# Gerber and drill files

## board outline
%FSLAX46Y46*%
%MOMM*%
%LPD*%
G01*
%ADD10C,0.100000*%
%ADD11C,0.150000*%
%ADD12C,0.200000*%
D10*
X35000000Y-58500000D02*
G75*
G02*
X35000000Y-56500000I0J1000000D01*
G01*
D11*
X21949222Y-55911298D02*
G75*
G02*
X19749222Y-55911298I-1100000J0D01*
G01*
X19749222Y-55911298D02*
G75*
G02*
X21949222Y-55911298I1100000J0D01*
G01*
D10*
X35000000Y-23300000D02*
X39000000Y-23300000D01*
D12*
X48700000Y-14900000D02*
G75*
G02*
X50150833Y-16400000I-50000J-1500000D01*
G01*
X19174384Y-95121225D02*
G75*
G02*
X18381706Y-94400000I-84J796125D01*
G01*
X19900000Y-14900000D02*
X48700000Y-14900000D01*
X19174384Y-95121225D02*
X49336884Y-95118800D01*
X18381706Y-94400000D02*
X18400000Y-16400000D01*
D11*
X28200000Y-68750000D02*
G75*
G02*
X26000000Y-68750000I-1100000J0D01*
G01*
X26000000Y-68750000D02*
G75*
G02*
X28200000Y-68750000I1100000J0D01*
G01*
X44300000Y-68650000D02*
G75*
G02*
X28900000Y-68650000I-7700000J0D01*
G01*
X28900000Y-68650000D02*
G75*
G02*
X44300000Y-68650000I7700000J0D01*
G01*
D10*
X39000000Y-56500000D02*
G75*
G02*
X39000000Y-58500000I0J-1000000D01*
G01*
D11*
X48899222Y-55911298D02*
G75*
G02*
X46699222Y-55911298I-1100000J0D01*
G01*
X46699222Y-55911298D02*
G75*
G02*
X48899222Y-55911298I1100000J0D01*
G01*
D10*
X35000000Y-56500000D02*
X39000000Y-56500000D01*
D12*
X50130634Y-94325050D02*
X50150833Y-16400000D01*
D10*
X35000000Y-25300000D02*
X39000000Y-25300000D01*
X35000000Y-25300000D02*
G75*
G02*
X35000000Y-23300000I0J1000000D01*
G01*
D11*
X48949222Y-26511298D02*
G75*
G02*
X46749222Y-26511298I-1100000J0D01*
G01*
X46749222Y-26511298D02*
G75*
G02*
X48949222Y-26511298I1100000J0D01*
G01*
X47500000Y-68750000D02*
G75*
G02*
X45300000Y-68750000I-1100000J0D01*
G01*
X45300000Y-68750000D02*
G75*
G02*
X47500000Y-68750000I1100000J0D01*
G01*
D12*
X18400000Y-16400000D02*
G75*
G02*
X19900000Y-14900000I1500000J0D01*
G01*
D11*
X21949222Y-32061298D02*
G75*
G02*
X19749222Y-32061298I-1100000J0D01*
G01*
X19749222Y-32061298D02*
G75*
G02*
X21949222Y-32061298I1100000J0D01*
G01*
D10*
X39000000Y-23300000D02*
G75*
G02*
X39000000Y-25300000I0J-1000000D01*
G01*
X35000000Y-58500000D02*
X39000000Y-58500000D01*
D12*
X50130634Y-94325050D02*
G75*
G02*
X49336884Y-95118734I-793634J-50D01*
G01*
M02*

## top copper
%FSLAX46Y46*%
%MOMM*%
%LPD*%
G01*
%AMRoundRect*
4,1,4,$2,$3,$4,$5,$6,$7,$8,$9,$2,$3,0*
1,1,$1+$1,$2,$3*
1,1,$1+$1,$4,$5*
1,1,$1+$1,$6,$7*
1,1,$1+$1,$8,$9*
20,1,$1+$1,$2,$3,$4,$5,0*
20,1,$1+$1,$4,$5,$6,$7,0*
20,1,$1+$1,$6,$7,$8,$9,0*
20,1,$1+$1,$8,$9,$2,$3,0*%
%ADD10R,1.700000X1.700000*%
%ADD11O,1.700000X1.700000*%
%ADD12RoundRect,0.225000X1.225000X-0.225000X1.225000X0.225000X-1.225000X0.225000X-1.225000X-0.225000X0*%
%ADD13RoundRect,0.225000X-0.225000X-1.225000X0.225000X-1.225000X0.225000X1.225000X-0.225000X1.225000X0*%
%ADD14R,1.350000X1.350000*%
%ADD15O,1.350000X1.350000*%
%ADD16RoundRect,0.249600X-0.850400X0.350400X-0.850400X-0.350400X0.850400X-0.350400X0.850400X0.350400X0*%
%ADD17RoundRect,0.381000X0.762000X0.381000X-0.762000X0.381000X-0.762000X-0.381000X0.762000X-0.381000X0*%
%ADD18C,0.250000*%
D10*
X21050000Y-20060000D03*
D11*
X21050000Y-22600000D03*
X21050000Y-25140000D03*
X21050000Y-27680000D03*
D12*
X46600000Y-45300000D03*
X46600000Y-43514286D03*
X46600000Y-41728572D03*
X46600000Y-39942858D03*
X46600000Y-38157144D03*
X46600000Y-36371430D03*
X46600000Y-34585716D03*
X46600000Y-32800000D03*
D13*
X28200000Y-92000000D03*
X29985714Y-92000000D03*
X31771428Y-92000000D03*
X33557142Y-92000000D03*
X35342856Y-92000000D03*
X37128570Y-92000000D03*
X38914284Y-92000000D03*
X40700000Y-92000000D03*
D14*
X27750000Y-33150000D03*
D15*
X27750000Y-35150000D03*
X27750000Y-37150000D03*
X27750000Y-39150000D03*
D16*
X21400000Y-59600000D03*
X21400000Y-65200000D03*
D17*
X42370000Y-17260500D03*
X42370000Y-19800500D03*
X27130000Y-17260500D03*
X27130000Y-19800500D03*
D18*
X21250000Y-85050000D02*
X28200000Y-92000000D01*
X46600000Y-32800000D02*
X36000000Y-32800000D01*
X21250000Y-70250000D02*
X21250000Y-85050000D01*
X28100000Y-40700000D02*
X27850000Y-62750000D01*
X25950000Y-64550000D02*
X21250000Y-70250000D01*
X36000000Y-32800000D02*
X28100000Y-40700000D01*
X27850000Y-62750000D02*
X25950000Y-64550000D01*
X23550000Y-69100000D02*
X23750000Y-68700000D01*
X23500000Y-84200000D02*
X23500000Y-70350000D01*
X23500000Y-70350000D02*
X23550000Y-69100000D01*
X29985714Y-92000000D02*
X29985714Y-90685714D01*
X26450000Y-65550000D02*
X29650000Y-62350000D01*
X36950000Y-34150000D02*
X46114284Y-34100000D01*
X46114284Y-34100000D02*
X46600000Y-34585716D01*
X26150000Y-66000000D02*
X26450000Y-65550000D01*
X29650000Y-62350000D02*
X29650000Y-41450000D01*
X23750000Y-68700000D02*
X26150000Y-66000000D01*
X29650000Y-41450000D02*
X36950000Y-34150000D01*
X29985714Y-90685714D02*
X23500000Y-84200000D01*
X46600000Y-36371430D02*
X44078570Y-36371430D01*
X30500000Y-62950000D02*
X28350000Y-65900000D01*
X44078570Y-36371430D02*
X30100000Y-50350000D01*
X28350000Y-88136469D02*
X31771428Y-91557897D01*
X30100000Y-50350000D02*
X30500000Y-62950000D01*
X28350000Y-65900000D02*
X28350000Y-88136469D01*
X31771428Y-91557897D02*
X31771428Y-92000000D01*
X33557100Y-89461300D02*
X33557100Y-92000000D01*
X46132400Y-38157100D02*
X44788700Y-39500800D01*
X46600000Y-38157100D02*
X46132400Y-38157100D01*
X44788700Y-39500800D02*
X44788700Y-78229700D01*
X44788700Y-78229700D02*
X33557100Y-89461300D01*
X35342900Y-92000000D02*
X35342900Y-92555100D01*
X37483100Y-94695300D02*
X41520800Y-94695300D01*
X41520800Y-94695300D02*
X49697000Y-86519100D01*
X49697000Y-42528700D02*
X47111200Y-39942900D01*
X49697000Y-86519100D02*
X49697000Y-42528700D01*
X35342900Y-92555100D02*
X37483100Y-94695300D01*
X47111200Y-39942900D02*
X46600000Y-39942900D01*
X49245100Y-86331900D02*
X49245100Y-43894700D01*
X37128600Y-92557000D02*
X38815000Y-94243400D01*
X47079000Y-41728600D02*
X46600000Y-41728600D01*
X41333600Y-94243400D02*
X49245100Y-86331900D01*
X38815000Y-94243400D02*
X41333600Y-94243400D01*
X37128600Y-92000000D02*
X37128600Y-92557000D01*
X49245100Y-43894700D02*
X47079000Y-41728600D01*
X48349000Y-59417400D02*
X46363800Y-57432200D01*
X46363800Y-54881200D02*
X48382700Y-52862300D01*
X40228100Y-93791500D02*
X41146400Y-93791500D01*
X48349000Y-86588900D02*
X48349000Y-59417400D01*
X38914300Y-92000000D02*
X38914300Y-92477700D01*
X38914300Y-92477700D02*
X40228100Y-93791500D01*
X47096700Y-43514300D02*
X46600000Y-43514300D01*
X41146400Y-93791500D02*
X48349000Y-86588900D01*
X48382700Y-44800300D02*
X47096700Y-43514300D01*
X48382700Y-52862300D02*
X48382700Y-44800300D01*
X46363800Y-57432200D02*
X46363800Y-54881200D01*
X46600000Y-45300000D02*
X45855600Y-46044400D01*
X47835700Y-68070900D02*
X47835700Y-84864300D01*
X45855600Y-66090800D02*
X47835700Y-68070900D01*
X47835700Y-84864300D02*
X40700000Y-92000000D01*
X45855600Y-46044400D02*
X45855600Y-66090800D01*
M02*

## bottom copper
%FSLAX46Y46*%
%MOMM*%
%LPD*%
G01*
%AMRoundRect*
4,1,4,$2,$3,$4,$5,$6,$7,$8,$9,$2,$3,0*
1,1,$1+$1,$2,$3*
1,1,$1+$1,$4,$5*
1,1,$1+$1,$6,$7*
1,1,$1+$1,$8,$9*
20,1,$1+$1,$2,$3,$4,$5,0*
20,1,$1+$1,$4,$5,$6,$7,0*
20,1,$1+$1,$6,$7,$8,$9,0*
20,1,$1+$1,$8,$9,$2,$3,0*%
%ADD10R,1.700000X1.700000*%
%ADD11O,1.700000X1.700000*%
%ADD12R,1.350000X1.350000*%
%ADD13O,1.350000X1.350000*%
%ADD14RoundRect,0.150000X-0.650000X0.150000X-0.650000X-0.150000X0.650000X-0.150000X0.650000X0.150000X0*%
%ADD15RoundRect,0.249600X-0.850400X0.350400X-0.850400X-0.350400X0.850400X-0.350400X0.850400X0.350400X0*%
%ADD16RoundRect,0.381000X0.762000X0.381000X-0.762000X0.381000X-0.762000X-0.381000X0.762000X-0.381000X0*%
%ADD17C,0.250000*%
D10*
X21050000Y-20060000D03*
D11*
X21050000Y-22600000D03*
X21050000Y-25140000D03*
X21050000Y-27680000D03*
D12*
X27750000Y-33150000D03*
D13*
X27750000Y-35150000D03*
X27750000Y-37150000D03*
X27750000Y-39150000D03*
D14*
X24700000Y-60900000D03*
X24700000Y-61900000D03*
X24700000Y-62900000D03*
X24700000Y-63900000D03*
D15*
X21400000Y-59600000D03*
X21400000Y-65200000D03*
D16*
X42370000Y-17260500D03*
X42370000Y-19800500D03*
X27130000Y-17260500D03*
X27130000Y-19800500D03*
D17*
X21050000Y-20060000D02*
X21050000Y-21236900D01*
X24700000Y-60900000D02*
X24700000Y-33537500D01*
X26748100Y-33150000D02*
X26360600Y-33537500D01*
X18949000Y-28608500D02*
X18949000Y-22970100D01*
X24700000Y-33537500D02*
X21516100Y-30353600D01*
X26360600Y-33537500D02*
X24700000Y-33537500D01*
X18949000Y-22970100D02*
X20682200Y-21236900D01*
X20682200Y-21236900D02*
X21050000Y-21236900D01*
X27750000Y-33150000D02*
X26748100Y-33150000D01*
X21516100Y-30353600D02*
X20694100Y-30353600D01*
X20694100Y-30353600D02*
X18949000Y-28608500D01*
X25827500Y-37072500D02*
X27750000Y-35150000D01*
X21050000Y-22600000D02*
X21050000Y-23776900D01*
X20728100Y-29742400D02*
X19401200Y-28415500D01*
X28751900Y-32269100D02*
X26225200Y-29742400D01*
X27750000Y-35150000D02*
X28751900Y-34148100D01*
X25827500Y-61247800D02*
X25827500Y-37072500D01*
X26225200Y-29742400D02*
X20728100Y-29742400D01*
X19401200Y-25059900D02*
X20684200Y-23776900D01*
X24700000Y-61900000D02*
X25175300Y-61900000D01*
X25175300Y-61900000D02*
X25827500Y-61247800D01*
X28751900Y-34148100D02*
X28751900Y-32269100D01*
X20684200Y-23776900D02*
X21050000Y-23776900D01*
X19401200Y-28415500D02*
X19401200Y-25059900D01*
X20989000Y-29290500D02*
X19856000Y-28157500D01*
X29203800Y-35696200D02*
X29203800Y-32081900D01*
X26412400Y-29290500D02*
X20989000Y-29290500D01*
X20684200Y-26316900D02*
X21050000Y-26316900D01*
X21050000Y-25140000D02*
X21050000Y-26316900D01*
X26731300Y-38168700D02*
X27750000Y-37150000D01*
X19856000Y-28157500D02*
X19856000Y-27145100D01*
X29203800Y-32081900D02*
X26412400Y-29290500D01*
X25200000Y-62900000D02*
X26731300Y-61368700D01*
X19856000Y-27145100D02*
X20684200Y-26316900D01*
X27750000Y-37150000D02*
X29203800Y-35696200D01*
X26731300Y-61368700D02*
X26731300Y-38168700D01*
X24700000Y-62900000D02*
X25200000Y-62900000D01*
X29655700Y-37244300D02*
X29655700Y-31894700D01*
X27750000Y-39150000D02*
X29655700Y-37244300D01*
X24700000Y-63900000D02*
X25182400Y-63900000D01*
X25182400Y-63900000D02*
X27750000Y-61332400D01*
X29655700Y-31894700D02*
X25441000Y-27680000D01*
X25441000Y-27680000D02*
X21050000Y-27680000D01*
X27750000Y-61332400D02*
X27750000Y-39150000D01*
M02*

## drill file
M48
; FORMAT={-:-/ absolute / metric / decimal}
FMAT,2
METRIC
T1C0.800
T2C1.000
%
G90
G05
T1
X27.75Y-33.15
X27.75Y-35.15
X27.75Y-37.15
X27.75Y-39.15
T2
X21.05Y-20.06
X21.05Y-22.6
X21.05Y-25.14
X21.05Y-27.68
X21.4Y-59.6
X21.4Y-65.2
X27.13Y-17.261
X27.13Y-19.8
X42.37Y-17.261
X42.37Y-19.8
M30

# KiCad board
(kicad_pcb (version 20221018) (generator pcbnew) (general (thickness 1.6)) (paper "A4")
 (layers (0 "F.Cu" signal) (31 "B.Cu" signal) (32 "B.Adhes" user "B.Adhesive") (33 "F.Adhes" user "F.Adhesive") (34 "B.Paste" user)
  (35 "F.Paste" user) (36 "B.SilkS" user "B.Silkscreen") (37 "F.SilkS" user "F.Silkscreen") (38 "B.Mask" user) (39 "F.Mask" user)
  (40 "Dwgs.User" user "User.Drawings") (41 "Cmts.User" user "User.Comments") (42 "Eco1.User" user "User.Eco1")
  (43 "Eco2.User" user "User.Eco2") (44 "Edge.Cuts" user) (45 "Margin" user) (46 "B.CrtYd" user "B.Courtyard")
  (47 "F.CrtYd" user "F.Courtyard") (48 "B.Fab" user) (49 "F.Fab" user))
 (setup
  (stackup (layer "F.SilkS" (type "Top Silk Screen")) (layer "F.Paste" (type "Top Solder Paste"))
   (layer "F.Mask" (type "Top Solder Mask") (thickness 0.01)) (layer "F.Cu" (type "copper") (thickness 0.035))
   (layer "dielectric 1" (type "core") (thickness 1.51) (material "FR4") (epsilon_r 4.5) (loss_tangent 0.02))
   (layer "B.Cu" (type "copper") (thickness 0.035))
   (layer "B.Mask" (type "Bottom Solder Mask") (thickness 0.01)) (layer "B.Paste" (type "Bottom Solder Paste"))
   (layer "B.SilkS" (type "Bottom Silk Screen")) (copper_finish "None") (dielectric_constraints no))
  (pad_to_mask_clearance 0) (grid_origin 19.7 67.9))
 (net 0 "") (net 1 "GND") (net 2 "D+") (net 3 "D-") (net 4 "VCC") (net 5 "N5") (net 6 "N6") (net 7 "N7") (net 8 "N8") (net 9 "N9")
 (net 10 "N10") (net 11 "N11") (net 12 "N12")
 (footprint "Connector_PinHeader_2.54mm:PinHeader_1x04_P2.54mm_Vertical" (layer "F.Cu") (at 21.05 20.06)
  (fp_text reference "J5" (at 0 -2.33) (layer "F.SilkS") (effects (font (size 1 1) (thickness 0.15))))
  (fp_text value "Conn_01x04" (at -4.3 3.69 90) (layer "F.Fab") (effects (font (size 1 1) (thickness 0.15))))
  (pad "1" thru_hole rect (at 0 0) (size 1.7 1.7) (drill 1) (layers "*.Cu" "*.Mask") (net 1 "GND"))
  (pad "2" thru_hole oval (at 0 2.54) (size 1.7 1.7) (drill 1) (layers "*.Cu" "*.Mask") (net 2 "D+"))
  (pad "3" thru_hole oval (at 0 5.08) (size 1.7 1.7) (drill 1) (layers "*.Cu" "*.Mask") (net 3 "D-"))
  (pad "4" thru_hole oval (at 0 7.62) (size 1.7 1.7) (drill 1) (layers "*.Cu" "*.Mask") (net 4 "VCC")))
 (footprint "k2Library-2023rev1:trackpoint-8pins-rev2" (layer "F.Cu") (at 44.1 38.55 90)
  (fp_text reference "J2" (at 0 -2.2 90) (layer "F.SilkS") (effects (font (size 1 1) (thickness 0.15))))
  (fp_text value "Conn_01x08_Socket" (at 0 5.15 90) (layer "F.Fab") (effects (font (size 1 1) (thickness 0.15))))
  (pad "1" smd roundrect (at -6.75 2.5 90) (size 0.9 2.9) (layers "F.Cu" "F.Paste" "F.Mask") (roundrect_rratio 0.25) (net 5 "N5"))
  (pad "2" smd roundrect (at -4.964286 2.5 90) (size 0.9 2.9) (layers "F.Cu" "F.Paste" "F.Mask") (roundrect_rratio 0.25) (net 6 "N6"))
  (pad "3" smd roundrect (at -3.178572 2.5 90) (size 0.9 2.9) (layers "F.Cu" "F.Paste" "F.Mask") (roundrect_rratio 0.25) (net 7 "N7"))
  (pad "4" smd roundrect (at -1.392858 2.5 90) (size 0.9 2.9) (layers "F.Cu" "F.Paste" "F.Mask") (roundrect_rratio 0.25) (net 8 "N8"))
  (pad "5" smd roundrect (at 0.392856 2.5 90) (size 0.9 2.9) (layers "F.Cu" "F.Paste" "F.Mask") (roundrect_rratio 0.25) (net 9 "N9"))
  (pad "6" smd roundrect (at 2.17857 2.5 90) (size 0.9 2.9) (layers "F.Cu" "F.Paste" "F.Mask") (roundrect_rratio 0.25) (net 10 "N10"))
  (pad "7" smd roundrect (at 3.964284 2.5 90) (size 0.9 2.9) (layers "F.Cu" "F.Paste" "F.Mask") (roundrect_rratio 0.25) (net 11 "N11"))
  (pad "8" smd roundrect (at 5.75 2.5 90) (size 0.9 2.9) (layers "F.Cu" "F.Paste" "F.Mask") (roundrect_rratio 0.25) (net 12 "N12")))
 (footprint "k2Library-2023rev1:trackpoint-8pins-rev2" (layer "F.Cu") (at 34.95 89.5)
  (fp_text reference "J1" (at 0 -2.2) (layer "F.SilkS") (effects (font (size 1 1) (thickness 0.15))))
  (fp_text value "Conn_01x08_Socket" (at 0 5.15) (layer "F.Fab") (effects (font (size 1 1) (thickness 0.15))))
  (pad "1" smd roundrect (at -6.75 2.5) (size 0.9 2.9) (layers "F.Cu" "F.Paste" "F.Mask") (roundrect_rratio 0.25) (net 12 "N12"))
  (pad "2" smd roundrect (at -4.964286 2.5) (size 0.9 2.9) (layers "F.Cu" "F.Paste" "F.Mask") (roundrect_rratio 0.25) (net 11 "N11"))
  (pad "3" smd roundrect (at -3.178572 2.5) (size 0.9 2.9) (layers "F.Cu" "F.Paste" "F.Mask") (roundrect_rratio 0.25) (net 10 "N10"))
  (pad "4" smd roundrect (at -1.392858 2.5) (size 0.9 2.9) (layers "F.Cu" "F.Paste" "F.Mask") (roundrect_rratio 0.25) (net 9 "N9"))
  (pad "5" smd roundrect (at 0.392856 2.5) (size 0.9 2.9) (layers "F.Cu" "F.Paste" "F.Mask") (roundrect_rratio 0.25) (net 8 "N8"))
  (pad "6" smd roundrect (at 2.17857 2.5) (size 0.9 2.9) (layers "F.Cu" "F.Paste" "F.Mask") (roundrect_rratio 0.25) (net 7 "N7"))
  (pad "7" smd roundrect (at 3.964284 2.5) (size 0.9 2.9) (layers "F.Cu" "F.Paste" "F.Mask") (roundrect_rratio 0.25) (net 6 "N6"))
  (pad "8" smd roundrect (at 5.75 2.5) (size 0.9 2.9) (layers "F.Cu" "F.Paste" "F.Mask") (roundrect_rratio 0.25) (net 5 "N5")))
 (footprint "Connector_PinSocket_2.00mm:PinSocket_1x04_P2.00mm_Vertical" (layer "B.Cu") (at 27.75 33.15 180)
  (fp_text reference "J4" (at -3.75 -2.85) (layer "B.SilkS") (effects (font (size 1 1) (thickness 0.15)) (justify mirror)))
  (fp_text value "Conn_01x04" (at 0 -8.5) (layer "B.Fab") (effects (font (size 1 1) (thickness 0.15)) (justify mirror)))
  (pad "1" thru_hole rect (at 0 0 180) (size 1.35 1.35) (drill 0.8) (layers "*.Cu" "*.Mask") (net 1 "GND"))
  (pad "2" thru_hole oval (at 0 -2 180) (size 1.35 1.35) (drill 0.8) (layers "*.Cu" "*.Mask") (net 2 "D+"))
  (pad "3" thru_hole oval (at 0 -4 180) (size 1.35 1.35) (drill 0.8) (layers "*.Cu" "*.Mask") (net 3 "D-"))
  (pad "4" thru_hole oval (at 0 -6 180) (size 1.35 1.35) (drill 0.8) (layers "*.Cu" "*.Mask") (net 4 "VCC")))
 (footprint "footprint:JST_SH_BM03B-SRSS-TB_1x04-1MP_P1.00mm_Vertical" (layer "B.Cu") (at 22.9 62.4 -90)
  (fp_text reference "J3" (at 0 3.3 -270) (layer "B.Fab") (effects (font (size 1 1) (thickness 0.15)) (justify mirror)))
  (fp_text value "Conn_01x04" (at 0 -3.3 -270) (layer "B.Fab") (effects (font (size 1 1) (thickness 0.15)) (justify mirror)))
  (pad "1" smd roundrect (at -1.5 -1.8 270) (size 0.6 1.6) (layers "B.Cu" "B.Paste" "B.Mask") (roundrect_rratio 0.25) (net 1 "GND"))
  (pad "2" smd roundrect (at -0.5 -1.8 270) (size 0.6 1.6) (layers "B.Cu" "B.Paste" "B.Mask") (roundrect_rratio 0.25) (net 2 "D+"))
  (pad "3" smd roundrect (at 0.5 -1.8 270) (size 0.6 1.6) (layers "B.Cu" "B.Paste" "B.Mask") (roundrect_rratio 0.25) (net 3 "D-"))
  (pad "4" smd roundrect (at 1.5 -1.8 270) (size 0.6 1.6) (layers "B.Cu" "B.Paste" "B.Mask") (roundrect_rratio 0.25) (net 4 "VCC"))
  (pad "MP" thru_hole roundrect (at -2.8 1.5 270) (size 1.2 2.2) (drill 1) (layers "*.Cu" "*.Mask") (roundrect_rratio 0.208))
  (pad "MP" thru_hole roundrect (at 2.8 1.5 270) (size 1.2 2.2) (drill 1) (layers "*.Cu" "*.Mask") (roundrect_rratio 0.208)))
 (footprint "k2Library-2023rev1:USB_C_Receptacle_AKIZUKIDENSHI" (layer "B.Cu") (at 34.75 22.6005 180)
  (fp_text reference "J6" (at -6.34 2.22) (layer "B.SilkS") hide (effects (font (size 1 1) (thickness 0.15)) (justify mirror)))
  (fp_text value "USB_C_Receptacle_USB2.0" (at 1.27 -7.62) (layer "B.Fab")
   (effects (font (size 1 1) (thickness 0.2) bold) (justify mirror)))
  (pad "1" thru_hole roundrect (at -7.62 5.34 180) (size 2.286 1.524) (drill 1) (layers "*.Cu" "*.Mask") (roundrect_rratio 0.25)
   (thermal_bridge_angle 45))
  (pad "2" thru_hole roundrect (at -7.62 2.8 180) (size 2.286 1.524) (drill 1) (layers "*.Cu" "*.Mask") (roundrect_rratio 0.25)
   (thermal_bridge_angle 45))
  (pad "3" thru_hole roundrect (at 7.62 5.34 180) (size 2.286 1.524) (drill 1) (layers "*.Cu" "*.Mask") (roundrect_rratio 0.25)
   (thermal_bridge_angle 45))
  (pad "4" thru_hole roundrect (at 7.62 2.8 180) (size 2.286 1.524) (drill 1) (layers "*.Cu" "*.Mask") (roundrect_rratio 0.25)
   (thermal_bridge_angle 45)))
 (gr_arc (start 35 58.5) (mid 34 57.5) (end 35 56.5) (stroke (width 0.1) (type default)) (layer "Edge.Cuts"))
 (gr_circle (center 20.849222 55.911298) (end 21.949222 55.911298) (stroke (width 0.15) (type default)) (fill none) (layer "Edge.Cuts"))
 (gr_line (start 35 23.3) (end 39 23.3) (stroke (width 0.1) (type default)) (layer "Edge.Cuts"))
 (gr_arc (start 48.7 14.9) (mid 49.728781 15.356578) (end 50.150833 16.4) (stroke (width 0.2) (type solid)) (layer "Edge.Cuts"))
 (gr_arc (start 19.174384 95.121225) (mid 18.638521 94.91396) (end 18.381706 94.4) (stroke (width 0.2) (type solid)) (layer "Edge.Cuts"))
 (gr_line (start 19.9 14.9) (end 48.7 14.9) (stroke (width 0.2) (type solid)) (layer "Edge.Cuts"))
 (gr_line (start 19.174384 95.121225) (end 49.336884 95.1188) (stroke (width 0.2) (type solid)) (layer "Edge.Cuts"))
 (gr_line (start 18.381706 94.4) (end 18.4 16.4) (stroke (width 0.2) (type solid)) (layer "Edge.Cuts"))
 (gr_circle (center 27.1 68.75) (end 28.2 68.75) (stroke (width 0.15) (type solid)) (fill none) (layer "Edge.Cuts"))
 (gr_circle (center 36.6 68.65) (end 44.3 68.65) (stroke (width 0.15) (type solid)) (fill none) (layer "Edge.Cuts"))
 (gr_arc (start 39 56.5) (mid 40 57.5) (end 39 58.5) (stroke (width 0.1) (type default)) (layer "Edge.Cuts"))
 (gr_circle (center 47.799222 55.911298) (end 48.899222 55.911298) (stroke (width 0.15) (type default)) (fill none) (layer "Edge.Cuts"))
 (gr_line (start 35 56.5) (end 39 56.5) (stroke (width 0.1) (type default)) (layer "Edge.Cuts"))
 (gr_line (start 50.130634 94.32505) (end 50.150833 16.4) (stroke (width 0.2) (type solid)) (layer "Edge.Cuts"))
 (gr_line (start 35 25.3) (end 39 25.3) (stroke (width 0.1) (type default)) (layer "Edge.Cuts"))
 (gr_arc (start 35 25.3) (mid 34 24.3) (end 35 23.3) (stroke (width 0.1) (type default)) (layer "Edge.Cuts"))
 (gr_circle (center 47.849222 26.511298) (end 48.949222 26.511298) (stroke (width 0.15) (type default)) (fill none) (layer "Edge.Cuts"))
 (gr_circle (center 46.4 68.75) (end 47.5 68.75) (stroke (width 0.15) (type solid)) (fill none) (layer "Edge.Cuts"))
 (gr_arc (start 18.4 16.4) (mid 18.83934 15.33934) (end 19.9 14.9) (stroke (width 0.2) (type solid)) (layer "Edge.Cuts"))
 (gr_circle (center 20.849222 32.061298) (end 21.949222 32.061298) (stroke (width 0.15) (type default)) (fill none) (layer "Edge.Cuts"))
 (gr_arc (start 39 23.3) (mid 40 24.3) (end 39 25.3) (stroke (width 0.1) (type default)) (layer "Edge.Cuts"))
 (gr_line (start 35 58.5) (end 39 58.5) (stroke (width 0.1) (type default)) (layer "Edge.Cuts"))
 (gr_arc (start 50.130634 94.32505) (mid 49.898174 94.88634) (end 49.336884 95.1188) (stroke (width 0.2) (type solid)) (layer "Edge.Cuts"))
 (segment (start 21.25 85.05) (end 28.2 92) (width 0.25) (layer "F.Cu") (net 12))
 (segment (start 46.6 32.8) (end 36 32.8) (width 0.25) (layer "F.Cu") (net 12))
 (segment (start 21.25 70.25) (end 21.25 85.05) (width 0.25) (layer "F.Cu") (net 12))
 (segment (start 28.1 40.7) (end 27.85 62.75) (width 0.25) (layer "F.Cu") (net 12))
 (segment (start 25.95 64.55) (end 21.25 70.25) (width 0.25) (layer "F.Cu") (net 12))
 (segment (start 36 32.8) (end 28.1 40.7) (width 0.25) (layer "F.Cu") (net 12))
 (segment (start 27.85 62.75) (end 25.95 64.55) (width 0.25) (layer "F.Cu") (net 12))
 (segment (start 23.55 69.1) (end 23.75 68.7) (width 0.25) (layer "F.Cu") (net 11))
 (segment (start 23.5 84.2) (end 23.5 70.35) (width 0.25) (layer "F.Cu") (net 11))
 (segment (start 23.5 70.35) (end 23.55 69.1) (width 0.25) (layer "F.Cu") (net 11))
 (segment (start 29.985714 92) (end 29.985714 90.685714) (width 0.25) (layer "F.Cu") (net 11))
 (segment (start 26.45 65.55) (end 29.65 62.35) (width 0.25) (layer "F.Cu") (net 11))
 (segment (start 36.95 34.15) (end 46.114284 34.1) (width 0.25) (layer "F.Cu") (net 11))
 (segment (start 46.114284 34.1) (end 46.6 34.585716) (width 0.25) (layer "F.Cu") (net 11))
 (segment (start 26.15 66) (end 26.45 65.55) (width 0.25) (layer "F.Cu") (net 11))
 (segment (start 29.65 62.35) (end 29.65 41.45) (width 0.25) (layer "F.Cu") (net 11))
 (segment (start 23.75 68.7) (end 26.15 66) (width 0.25) (layer "F.Cu") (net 11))
 (segment (start 29.65 41.45) (end 36.95 34.15) (width 0.25) (layer "F.Cu") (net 11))
 (segment (start 29.985714 90.685714) (end 23.5 84.2) (width 0.25) (layer "F.Cu") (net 11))
 (segment (start 46.6 36.37143) (end 44.07857 36.37143) (width 0.25) (layer "F.Cu") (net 10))
 (segment (start 30.5 62.95) (end 28.35 65.9) (width 0.25) (layer "F.Cu") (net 10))
 (segment (start 44.07857 36.37143) (end 30.1 50.35) (width 0.25) (layer "F.Cu") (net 10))
 (segment (start 28.35 88.136469) (end 31.771428 91.557897) (width 0.25) (layer "F.Cu") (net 10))
 (segment (start 30.1 50.35) (end 30.5 62.95) (width 0.25) (layer "F.Cu") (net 10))
 (segment (start 28.35 65.9) (end 28.35 88.136469) (width 0.25) (layer "F.Cu") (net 10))
 (segment (start 31.771428 91.557897) (end 31.771428 92) (width 0.25) (layer "F.Cu") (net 10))
 (segment (start 33.5571 89.4613) (end 33.5571 92) (width 0.25) (layer "F.Cu") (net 9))
 (segment (start 46.1324 38.1571) (end 44.7887 39.5008) (width 0.25) (layer "F.Cu") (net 9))
 (segment (start 46.6 38.1571) (end 46.1324 38.1571) (width 0.25) (layer "F.Cu") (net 9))
 (segment (start 44.7887 39.5008) (end 44.7887 78.2297) (width 0.25) (layer "F.Cu") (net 9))
 (segment (start 44.7887 78.2297) (end 33.5571 89.4613) (width 0.25) (layer "F.Cu") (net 9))
 (segment (start 35.3429 92) (end 35.3429 92.5551) (width 0.25) (layer "F.Cu") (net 8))
 (segment (start 37.4831 94.6953) (end 41.5208 94.6953) (width 0.25) (layer "F.Cu") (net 8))
 (segment (start 41.5208 94.6953) (end 49.697 86.5191) (width 0.25) (layer "F.Cu") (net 8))
 (segment (start 49.697 42.5287) (end 47.1112 39.9429) (width 0.25) (layer "F.Cu") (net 8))
 (segment (start 49.697 86.5191) (end 49.697 42.5287) (width 0.25) (layer "F.Cu") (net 8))
 (segment (start 35.3429 92.5551) (end 37.4831 94.6953) (width 0.25) (layer "F.Cu") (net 8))
 (segment (start 47.1112 39.9429) (end 46.6 39.9429) (width 0.25) (layer "F.Cu") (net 8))
 (segment (start 49.2451 86.3319) (end 49.2451 43.8947) (width 0.25) (layer "F.Cu") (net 7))
 (segment (start 37.1286 92.557) (end 38.815 94.2434) (width 0.25) (layer "F.Cu") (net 7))
 (segment (start 47.079 41.7286) (end 46.6 41.7286) (width 0.25) (layer "F.Cu") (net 7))
 (segment (start 41.3336 94.2434) (end 49.2451 86.3319) (width 0.25) (layer "F.Cu") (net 7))
 (segment (start 38.815 94.2434) (end 41.3336 94.2434) (width 0.25) (layer "F.Cu") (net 7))
 (segment (start 37.1286 92) (end 37.1286 92.557) (width 0.25) (layer "F.Cu") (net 7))
 (segment (start 49.2451 43.8947) (end 47.079 41.7286) (width 0.25) (layer "F.Cu") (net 7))
 (segment (start 48.349 59.4174) (end 46.3638 57.4322) (width 0.25) (layer "F.Cu") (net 6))
 (segment (start 46.3638 54.8812) (end 48.3827 52.8623) (width 0.25) (layer "F.Cu") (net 6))
 (segment (start 40.2281 93.7915) (end 41.1464 93.7915) (width 0.25) (layer "F.Cu") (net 6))
 (segment (start 48.349 86.5889) (end 48.349 59.4174) (width 0.25) (layer "F.Cu") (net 6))
 (segment (start 38.9143 92) (end 38.9143 92.4777) (width 0.25) (layer "F.Cu") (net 6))
 (segment (start 38.9143 92.4777) (end 40.2281 93.7915) (width 0.25) (layer "F.Cu") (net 6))
 (segment (start 47.0967 43.5143) (end 46.6 43.5143) (width 0.25) (layer "F.Cu") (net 6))
 (segment (start 41.1464 93.7915) (end 48.349 86.5889) (width 0.25) (layer "F.Cu") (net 6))
 (segment (start 48.3827 44.8003) (end 47.0967 43.5143) (width 0.25) (layer "F.Cu") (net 6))
 (segment (start 48.3827 52.8623) (end 48.3827 44.8003) (width 0.25) (layer "F.Cu") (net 6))
 (segment (start 46.3638 57.4322) (end 46.3638 54.8812) (width 0.25) (layer "F.Cu") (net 6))
 (segment (start 46.6 45.3) (end 45.8556 46.0444) (width 0.25) (layer "F.Cu") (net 5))
 (segment (start 47.8357 68.0709) (end 47.8357 84.8643) (width 0.25) (layer "F.Cu") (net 5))
 (segment (start 45.8556 66.0908) (end 47.8357 68.0709) (width 0.25) (layer "F.Cu") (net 5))
 (segment (start 47.8357 84.8643) (end 40.7 92) (width 0.25) (layer "F.Cu") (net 5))
 (segment (start 45.8556 46.0444) (end 45.8556 66.0908) (width 0.25) (layer "F.Cu") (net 5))
 (segment (start 21.05 20.06) (end 21.05 21.2369) (width 0.25) (layer "B.Cu") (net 1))
 (segment (start 24.7 60.9) (end 24.7 33.5375) (width 0.25) (layer "B.Cu") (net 1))
 (segment (start 26.7481 33.15) (end 26.3606 33.5375) (width 0.25) (layer "B.Cu") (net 1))
 (segment (start 18.949 28.6085) (end 18.949 22.9701) (width 0.25) (layer "B.Cu") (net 1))
 (segment (start 24.7 33.5375) (end 21.5161 30.3536) (width 0.25) (layer "B.Cu") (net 1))
 (segment (start 26.3606 33.5375) (end 24.7 33.5375) (width 0.25) (layer "B.Cu") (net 1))
 (segment (start 18.949 22.9701) (end 20.6822 21.2369) (width 0.25) (layer "B.Cu") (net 1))
 (segment (start 20.6822 21.2369) (end 21.05 21.2369) (width 0.25) (layer "B.Cu") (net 1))
 (segment (start 27.75 33.15) (end 26.7481 33.15) (width 0.25) (layer "B.Cu") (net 1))
 (segment (start 21.5161 30.3536) (end 20.6941 30.3536) (width 0.25) (layer "B.Cu") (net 1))
 (segment (start 20.6941 30.3536) (end 18.949 28.6085) (width 0.25) (layer "B.Cu") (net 1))
 (segment (start 25.8275 37.0725) (end 27.75 35.15) (width 0.25) (layer "B.Cu") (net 2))
 (segment (start 21.05 22.6) (end 21.05 23.7769) (width 0.25) (layer "B.Cu") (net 2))
 (segment (start 20.7281 29.7424) (end 19.4012 28.4155) (width 0.25) (layer "B.Cu") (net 2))
 (segment (start 28.7519 32.2691) (end 26.2252 29.7424) (width 0.25) (layer "B.Cu") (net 2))
 (segment (start 27.75 35.15) (end 28.7519 34.1481) (width 0.25) (layer "B.Cu") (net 2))
 (segment (start 25.8275 61.2478) (end 25.8275 37.0725) (width 0.25) (layer "B.Cu") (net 2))
 (segment (start 26.2252 29.7424) (end 20.7281 29.7424) (width 0.25) (layer "B.Cu") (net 2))
 (segment (start 19.4012 25.0599) (end 20.6842 23.7769) (width 0.25) (layer "B.Cu") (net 2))
 (segment (start 24.7 61.9) (end 25.1753 61.9) (width 0.25) (layer "B.Cu") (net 2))
 (segment (start 25.1753 61.9) (end 25.8275 61.2478) (width 0.25) (layer "B.Cu") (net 2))
 (segment (start 28.7519 34.1481) (end 28.7519 32.2691) (width 0.25) (layer "B.Cu") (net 2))
 (segment (start 20.6842 23.7769) (end 21.05 23.7769) (width 0.25) (layer "B.Cu") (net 2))
 (segment (start 19.4012 28.4155) (end 19.4012 25.0599) (width 0.25) (layer "B.Cu") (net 2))
 (segment (start 20.989 29.2905) (end 19.856 28.1575) (width 0.25) (layer "B.Cu") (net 3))
 (segment (start 29.2038 35.6962) (end 29.2038 32.0819) (width 0.25) (layer "B.Cu") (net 3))
 (segment (start 26.4124 29.2905) (end 20.989 29.2905) (width 0.25) (layer "B.Cu") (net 3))
 (segment (start 20.6842 26.3169) (end 21.05 26.3169) (width 0.25) (layer "B.Cu") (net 3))
 (segment (start 21.05 25.14) (end 21.05 26.3169) (width 0.25) (layer "B.Cu") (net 3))
 (segment (start 26.7313 38.1687) (end 27.75 37.15) (width 0.25) (layer "B.Cu") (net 3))
 (segment (start 19.856 28.1575) (end 19.856 27.1451) (width 0.25) (layer "B.Cu") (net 3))
 (segment (start 29.2038 32.0819) (end 26.4124 29.2905) (width 0.25) (layer "B.Cu") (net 3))
 (segment (start 25.2 62.9) (end 26.7313 61.3687) (width 0.25) (layer "B.Cu") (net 3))
 (segment (start 19.856 27.1451) (end 20.6842 26.3169) (width 0.25) (layer "B.Cu") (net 3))
 (segment (start 27.75 37.15) (end 29.2038 35.6962) (width 0.25) (layer "B.Cu") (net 3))
 (segment (start 26.7313 61.3687) (end 26.7313 38.1687) (width 0.25) (layer "B.Cu") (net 3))
 (segment (start 24.7 62.9) (end 25.2 62.9) (width 0.25) (layer "B.Cu") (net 3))
 (segment (start 29.6557 37.2443) (end 29.6557 31.8947) (width 0.25) (layer "B.Cu") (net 4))
 (segment (start 27.75 39.15) (end 29.6557 37.2443) (width 0.25) (layer "B.Cu") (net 4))
 (segment (start 24.7 63.9) (end 25.1824 63.9) (width 0.25) (layer "B.Cu") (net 4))
 (segment (start 25.1824 63.9) (end 27.75 61.3324) (width 0.25) (layer "B.Cu") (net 4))
 (segment (start 29.6557 31.8947) (end 25.441 27.68) (width 0.25) (layer "B.Cu") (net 4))
 (segment (start 25.441 27.68) (end 21.05 27.68) (width 0.25) (layer "B.Cu") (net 4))
 (segment (start 27.75 61.3324) (end 27.75 39.15) (width 0.25) (layer "B.Cu") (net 4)))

